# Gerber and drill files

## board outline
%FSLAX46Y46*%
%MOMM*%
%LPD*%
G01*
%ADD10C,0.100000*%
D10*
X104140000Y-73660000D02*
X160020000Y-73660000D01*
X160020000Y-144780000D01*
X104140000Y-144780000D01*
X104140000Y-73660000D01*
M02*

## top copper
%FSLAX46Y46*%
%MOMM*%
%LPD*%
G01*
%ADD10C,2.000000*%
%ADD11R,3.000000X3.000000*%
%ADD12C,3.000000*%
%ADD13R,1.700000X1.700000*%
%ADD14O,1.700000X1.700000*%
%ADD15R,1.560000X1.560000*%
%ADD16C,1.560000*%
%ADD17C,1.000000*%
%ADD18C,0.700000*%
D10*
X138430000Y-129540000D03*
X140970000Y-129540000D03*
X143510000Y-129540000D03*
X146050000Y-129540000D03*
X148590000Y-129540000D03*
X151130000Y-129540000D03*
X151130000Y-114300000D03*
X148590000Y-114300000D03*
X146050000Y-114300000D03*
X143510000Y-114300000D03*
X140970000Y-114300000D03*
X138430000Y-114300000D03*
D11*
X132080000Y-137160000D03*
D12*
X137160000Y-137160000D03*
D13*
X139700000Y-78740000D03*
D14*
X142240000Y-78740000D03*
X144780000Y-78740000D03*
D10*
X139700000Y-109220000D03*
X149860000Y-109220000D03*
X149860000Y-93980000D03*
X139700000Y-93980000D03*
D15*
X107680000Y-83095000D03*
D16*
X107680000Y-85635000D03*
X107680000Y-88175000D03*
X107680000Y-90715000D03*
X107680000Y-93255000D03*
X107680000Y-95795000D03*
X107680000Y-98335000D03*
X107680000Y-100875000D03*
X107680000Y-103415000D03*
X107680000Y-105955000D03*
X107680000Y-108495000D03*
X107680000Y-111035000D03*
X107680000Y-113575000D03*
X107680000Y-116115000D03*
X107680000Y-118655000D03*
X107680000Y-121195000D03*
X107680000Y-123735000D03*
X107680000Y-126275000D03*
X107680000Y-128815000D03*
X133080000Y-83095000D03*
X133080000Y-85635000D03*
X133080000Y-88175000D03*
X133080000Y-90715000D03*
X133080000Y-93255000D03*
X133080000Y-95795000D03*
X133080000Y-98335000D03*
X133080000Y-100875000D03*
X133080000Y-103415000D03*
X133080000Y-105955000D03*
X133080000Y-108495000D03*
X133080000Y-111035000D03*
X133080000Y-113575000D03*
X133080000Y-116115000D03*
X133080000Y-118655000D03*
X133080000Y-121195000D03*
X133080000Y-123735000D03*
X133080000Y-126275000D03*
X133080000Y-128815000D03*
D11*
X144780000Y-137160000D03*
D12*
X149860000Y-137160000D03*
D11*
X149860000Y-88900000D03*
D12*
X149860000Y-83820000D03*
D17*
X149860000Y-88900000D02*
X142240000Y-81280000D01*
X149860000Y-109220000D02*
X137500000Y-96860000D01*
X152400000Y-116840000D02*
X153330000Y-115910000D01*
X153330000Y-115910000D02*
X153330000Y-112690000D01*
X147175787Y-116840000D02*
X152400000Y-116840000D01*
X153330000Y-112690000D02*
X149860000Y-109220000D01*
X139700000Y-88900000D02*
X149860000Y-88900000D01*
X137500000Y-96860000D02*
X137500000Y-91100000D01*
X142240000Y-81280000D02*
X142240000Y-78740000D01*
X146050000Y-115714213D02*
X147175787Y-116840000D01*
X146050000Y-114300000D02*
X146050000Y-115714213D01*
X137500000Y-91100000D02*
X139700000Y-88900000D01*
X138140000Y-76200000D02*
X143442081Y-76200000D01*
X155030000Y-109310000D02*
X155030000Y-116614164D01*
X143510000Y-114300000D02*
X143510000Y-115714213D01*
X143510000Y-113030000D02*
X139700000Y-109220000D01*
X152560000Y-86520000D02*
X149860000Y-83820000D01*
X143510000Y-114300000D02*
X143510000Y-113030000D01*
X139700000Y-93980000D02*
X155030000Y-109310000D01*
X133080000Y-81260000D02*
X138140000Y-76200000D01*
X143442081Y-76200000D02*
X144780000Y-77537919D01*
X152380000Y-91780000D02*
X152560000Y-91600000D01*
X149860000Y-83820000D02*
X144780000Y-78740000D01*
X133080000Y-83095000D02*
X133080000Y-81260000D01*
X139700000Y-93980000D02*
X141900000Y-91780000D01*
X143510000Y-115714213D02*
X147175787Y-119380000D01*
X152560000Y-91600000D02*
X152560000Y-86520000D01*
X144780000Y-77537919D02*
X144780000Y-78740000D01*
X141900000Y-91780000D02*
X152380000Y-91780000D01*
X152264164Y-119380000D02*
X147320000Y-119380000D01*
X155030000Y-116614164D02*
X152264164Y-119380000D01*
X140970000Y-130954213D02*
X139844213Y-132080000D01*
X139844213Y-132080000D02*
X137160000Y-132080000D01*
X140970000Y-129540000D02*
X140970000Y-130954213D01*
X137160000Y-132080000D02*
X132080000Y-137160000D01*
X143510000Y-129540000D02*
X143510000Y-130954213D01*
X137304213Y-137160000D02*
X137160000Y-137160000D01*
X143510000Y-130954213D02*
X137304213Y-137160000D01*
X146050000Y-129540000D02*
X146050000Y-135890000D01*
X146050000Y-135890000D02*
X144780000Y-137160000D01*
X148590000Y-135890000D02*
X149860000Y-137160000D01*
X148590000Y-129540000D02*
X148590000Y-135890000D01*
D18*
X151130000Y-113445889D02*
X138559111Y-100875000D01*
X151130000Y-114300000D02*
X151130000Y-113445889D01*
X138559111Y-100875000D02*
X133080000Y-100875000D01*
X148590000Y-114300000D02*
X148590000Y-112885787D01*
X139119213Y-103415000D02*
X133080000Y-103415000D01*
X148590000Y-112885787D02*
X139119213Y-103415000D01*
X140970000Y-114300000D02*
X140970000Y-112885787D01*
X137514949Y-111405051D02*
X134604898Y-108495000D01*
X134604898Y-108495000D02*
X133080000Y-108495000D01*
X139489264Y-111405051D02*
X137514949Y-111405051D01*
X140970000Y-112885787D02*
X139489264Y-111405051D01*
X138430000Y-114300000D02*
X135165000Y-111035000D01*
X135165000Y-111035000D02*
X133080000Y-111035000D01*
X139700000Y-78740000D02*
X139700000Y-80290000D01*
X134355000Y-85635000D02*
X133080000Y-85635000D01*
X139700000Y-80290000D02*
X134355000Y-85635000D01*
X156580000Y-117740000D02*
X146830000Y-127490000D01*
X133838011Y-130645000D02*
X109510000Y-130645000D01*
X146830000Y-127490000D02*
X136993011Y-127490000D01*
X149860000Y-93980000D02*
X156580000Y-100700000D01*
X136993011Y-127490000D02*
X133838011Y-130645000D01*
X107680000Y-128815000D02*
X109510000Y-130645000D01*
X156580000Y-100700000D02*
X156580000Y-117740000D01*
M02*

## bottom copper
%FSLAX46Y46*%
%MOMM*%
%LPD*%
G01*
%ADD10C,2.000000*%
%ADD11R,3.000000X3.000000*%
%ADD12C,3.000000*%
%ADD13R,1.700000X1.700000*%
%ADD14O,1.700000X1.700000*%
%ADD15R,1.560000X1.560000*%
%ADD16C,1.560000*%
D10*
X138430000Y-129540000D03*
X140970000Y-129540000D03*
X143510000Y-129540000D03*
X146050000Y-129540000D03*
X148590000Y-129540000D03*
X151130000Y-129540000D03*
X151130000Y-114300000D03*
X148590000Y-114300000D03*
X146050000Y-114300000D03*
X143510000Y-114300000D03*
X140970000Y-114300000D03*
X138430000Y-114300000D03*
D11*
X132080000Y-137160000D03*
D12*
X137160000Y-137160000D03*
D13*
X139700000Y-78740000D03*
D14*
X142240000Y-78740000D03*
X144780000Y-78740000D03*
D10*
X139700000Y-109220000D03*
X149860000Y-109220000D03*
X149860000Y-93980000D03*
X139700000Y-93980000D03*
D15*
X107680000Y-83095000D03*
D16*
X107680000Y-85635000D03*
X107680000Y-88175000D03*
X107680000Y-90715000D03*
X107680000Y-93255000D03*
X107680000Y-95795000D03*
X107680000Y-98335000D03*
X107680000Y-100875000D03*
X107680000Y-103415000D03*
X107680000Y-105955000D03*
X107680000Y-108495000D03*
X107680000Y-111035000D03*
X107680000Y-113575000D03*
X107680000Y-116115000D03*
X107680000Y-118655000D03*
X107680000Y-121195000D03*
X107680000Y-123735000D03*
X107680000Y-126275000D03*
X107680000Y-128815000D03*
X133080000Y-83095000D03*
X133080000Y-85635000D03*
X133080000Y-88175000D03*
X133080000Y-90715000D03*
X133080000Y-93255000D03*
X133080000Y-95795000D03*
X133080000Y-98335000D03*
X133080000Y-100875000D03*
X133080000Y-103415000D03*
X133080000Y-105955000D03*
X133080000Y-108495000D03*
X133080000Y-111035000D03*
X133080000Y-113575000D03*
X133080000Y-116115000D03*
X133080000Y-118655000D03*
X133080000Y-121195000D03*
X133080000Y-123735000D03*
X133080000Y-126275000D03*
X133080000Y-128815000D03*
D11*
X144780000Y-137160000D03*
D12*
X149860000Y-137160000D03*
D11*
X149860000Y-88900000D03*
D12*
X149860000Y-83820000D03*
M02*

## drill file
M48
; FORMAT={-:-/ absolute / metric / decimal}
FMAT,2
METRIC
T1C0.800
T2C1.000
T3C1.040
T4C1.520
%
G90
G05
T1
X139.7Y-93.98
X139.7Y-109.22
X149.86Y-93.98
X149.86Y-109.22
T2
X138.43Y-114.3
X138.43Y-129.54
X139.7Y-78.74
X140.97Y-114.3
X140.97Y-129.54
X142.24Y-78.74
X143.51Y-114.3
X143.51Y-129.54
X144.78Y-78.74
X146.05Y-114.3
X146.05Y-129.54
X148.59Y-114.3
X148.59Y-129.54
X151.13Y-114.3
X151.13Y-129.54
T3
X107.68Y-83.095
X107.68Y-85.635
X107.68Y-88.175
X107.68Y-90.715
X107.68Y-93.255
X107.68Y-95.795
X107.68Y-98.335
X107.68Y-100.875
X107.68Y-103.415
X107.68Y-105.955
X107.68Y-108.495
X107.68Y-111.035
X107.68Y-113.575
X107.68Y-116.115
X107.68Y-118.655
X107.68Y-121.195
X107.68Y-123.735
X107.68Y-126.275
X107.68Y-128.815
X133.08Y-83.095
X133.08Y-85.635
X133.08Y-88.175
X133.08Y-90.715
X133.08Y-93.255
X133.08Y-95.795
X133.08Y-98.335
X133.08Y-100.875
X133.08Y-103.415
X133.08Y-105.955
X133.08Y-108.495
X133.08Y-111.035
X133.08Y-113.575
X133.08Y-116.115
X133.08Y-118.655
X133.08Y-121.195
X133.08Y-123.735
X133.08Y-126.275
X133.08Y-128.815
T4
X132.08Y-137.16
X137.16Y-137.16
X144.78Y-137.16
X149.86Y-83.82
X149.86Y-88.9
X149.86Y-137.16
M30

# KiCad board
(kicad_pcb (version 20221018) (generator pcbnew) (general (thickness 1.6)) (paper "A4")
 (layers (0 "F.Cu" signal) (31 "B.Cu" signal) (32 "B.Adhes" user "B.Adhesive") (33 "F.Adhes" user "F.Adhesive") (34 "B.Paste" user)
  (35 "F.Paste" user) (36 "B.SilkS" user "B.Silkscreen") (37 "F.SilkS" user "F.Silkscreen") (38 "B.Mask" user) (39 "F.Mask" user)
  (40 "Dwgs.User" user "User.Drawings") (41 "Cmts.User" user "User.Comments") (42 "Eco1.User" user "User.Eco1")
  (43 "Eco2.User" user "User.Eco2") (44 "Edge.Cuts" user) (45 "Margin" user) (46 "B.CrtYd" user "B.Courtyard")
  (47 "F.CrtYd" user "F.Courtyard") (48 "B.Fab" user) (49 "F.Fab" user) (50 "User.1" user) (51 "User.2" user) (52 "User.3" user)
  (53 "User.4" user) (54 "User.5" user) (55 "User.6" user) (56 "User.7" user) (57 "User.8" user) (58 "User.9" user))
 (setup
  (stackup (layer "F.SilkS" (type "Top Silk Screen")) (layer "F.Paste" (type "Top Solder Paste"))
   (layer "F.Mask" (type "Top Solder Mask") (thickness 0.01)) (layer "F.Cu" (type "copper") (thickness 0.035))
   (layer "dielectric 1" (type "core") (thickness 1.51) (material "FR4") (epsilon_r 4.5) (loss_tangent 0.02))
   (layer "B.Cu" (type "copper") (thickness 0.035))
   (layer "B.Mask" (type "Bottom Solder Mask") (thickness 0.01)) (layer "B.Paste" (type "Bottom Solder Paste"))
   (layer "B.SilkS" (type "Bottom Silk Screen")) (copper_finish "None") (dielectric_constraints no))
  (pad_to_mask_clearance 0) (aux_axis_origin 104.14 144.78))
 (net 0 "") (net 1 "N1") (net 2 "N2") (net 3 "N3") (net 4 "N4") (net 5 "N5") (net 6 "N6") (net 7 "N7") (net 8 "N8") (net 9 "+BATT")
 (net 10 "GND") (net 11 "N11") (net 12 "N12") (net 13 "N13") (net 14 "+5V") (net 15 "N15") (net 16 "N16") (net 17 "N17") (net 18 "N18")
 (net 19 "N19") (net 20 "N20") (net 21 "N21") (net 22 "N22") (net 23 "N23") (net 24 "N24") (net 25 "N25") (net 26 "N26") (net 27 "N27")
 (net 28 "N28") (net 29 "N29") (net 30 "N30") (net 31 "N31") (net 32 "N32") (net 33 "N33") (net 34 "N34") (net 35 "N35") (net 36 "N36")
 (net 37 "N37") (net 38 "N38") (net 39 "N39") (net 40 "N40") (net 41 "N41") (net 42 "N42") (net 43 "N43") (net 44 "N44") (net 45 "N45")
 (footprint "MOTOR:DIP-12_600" (layer "F.Cu") (at 144.78 121.92)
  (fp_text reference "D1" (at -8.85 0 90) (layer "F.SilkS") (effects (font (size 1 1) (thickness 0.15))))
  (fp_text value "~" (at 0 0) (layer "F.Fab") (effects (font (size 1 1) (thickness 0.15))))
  (pad "1" thru_hole circle (at -6.35 7.62) (size 2 2) (drill 1) (layers "*.Cu" "*.Mask") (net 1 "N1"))
  (pad "2" thru_hole circle (at -3.81 7.62) (size 2 2) (drill 1) (layers "*.Cu" "*.Mask") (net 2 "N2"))
  (pad "3" thru_hole circle (at -1.27 7.62) (size 2 2) (drill 1) (layers "*.Cu" "*.Mask") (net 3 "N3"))
  (pad "4" thru_hole circle (at 1.27 7.62) (size 2 2) (drill 1) (layers "*.Cu" "*.Mask") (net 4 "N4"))
  (pad "5" thru_hole circle (at 3.81 7.62) (size 2 2) (drill 1) (layers "*.Cu" "*.Mask") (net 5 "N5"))
  (pad "6" thru_hole circle (at 6.35 7.62) (size 2 2) (drill 1) (layers "*.Cu" "*.Mask") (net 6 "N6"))
  (pad "7" thru_hole circle (at 6.35 -7.62) (size 2 2) (drill 1) (layers "*.Cu" "*.Mask") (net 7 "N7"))
  (pad "8" thru_hole circle (at 3.81 -7.62) (size 2 2) (drill 1) (layers "*.Cu" "*.Mask") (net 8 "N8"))
  (pad "9" thru_hole circle (at 1.27 -7.62) (size 2 2) (drill 1) (layers "*.Cu" "*.Mask") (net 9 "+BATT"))
  (pad "10" thru_hole circle (at -1.27 -7.62) (size 2 2) (drill 1) (layers "*.Cu" "*.Mask") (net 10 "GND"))
  (pad "11" thru_hole circle (at -3.81 -7.62) (size 2 2) (drill 1) (layers "*.Cu" "*.Mask") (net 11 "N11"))
  (pad "12" thru_hole circle (at -6.35 -7.62) (size 2 2) (drill 1) (layers "*.Cu" "*.Mask") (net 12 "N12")))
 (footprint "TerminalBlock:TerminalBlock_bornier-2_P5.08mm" (layer "F.Cu") (at 132.08 137.16)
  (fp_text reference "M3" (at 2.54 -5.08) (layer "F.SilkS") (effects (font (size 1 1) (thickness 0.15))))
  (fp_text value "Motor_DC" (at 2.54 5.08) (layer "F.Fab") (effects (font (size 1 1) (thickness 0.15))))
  (pad "1" thru_hole rect (at 0 0) (size 3 3) (drill 1.52) (layers "*.Cu" "*.Mask") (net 2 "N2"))
  (pad "2" thru_hole circle (at 5.08 0) (size 3 3) (drill 1.52) (layers "*.Cu" "*.Mask") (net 3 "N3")))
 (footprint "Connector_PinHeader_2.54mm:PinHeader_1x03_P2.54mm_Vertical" (layer "F.Cu") (at 139.7 78.74 90)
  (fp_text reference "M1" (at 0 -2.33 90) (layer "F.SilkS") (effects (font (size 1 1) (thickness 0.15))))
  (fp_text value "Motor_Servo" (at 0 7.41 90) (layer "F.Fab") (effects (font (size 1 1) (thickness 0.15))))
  (pad "1" thru_hole rect (at 0 0 90) (size 1.7 1.7) (drill 1) (layers "*.Cu" "*.Mask") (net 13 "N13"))
  (pad "2" thru_hole oval (at 0 2.54 90) (size 1.7 1.7) (drill 1) (layers "*.Cu" "*.Mask") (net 9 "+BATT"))
  (pad "3" thru_hole oval (at 0 5.08 90) (size 1.7 1.7) (drill 1) (layers "*.Cu" "*.Mask") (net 10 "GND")))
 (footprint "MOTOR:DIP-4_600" (layer "F.Cu") (at 144.78 101.6)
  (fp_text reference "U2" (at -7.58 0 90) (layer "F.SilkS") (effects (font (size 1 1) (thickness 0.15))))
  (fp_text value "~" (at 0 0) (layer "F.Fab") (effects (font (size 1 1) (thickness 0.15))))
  (pad "1" thru_hole circle (at -5.08 7.62) (size 2 2) (drill 0.8) (layers "*.Cu" "*.Mask") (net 10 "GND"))
  (pad "2" thru_hole circle (at 5.08 7.62) (size 2 2) (drill 0.8) (layers "*.Cu" "*.Mask") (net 9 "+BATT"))
  (pad "3" thru_hole circle (at 5.08 -7.62) (size 2 2) (drill 0.8) (layers "*.Cu" "*.Mask") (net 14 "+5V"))
  (pad "4" thru_hole circle (at -5.08 -7.62) (size 2 2) (drill 0.8) (layers "*.Cu" "*.Mask") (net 10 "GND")))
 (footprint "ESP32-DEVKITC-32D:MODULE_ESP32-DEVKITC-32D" (layer "F.Cu") (at 120.38 102.855)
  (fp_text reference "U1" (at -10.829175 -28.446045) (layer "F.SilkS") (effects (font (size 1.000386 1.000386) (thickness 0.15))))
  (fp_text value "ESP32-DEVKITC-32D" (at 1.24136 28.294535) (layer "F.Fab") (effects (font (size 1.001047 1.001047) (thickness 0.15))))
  (pad "J2-1" thru_hole rect (at -12.7 -19.76) (size 1.56 1.56) (drill 1.04) (layers "*.Cu" "*.Mask") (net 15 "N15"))
  (pad "J2-2" thru_hole circle (at -12.7 -17.22) (size 1.56 1.56) (drill 1.04) (layers "*.Cu" "*.Mask") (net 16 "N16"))
  (pad "J2-3" thru_hole circle (at -12.7 -14.68) (size 1.56 1.56) (drill 1.04) (layers "*.Cu" "*.Mask") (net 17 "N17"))
  (pad "J2-4" thru_hole circle (at -12.7 -12.14) (size 1.56 1.56) (drill 1.04) (layers "*.Cu" "*.Mask") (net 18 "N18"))
  (pad "J2-5" thru_hole circle (at -12.7 -9.6) (size 1.56 1.56) (drill 1.04) (layers "*.Cu" "*.Mask") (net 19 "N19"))
  (pad "J2-6" thru_hole circle (at -12.7 -7.06) (size 1.56 1.56) (drill 1.04) (layers "*.Cu" "*.Mask") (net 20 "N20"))
  (pad "J2-7" thru_hole circle (at -12.7 -4.52) (size 1.56 1.56) (drill 1.04) (layers "*.Cu" "*.Mask") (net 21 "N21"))
  (pad "J2-8" thru_hole circle (at -12.7 -1.98) (size 1.56 1.56) (drill 1.04) (layers "*.Cu" "*.Mask") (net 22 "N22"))
  (pad "J2-9" thru_hole circle (at -12.7 0.56) (size 1.56 1.56) (drill 1.04) (layers "*.Cu" "*.Mask") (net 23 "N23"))
  (pad "J2-10" thru_hole circle (at -12.7 3.1) (size 1.56 1.56) (drill 1.04) (layers "*.Cu" "*.Mask") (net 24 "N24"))
  (pad "J2-11" thru_hole circle (at -12.7 5.64) (size 1.56 1.56) (drill 1.04) (layers "*.Cu" "*.Mask") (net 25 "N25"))
  (pad "J2-12" thru_hole circle (at -12.7 8.18) (size 1.56 1.56) (drill 1.04) (layers "*.Cu" "*.Mask") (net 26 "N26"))
  (pad "J2-13" thru_hole circle (at -12.7 10.72) (size 1.56 1.56) (drill 1.04) (layers "*.Cu" "*.Mask") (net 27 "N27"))
  (pad "J2-14" thru_hole circle (at -12.7 13.26) (size 1.56 1.56) (drill 1.04) (layers "*.Cu" "*.Mask") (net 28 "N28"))
  (pad "J2-15" thru_hole circle (at -12.7 15.8) (size 1.56 1.56) (drill 1.04) (layers "*.Cu" "*.Mask") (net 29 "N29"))
  (pad "J2-16" thru_hole circle (at -12.7 18.34) (size 1.56 1.56) (drill 1.04) (layers "*.Cu" "*.Mask") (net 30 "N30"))
  (pad "J2-17" thru_hole circle (at -12.7 20.88) (size 1.56 1.56) (drill 1.04) (layers "*.Cu" "*.Mask") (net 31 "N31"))
  (pad "J2-18" thru_hole circle (at -12.7 23.42) (size 1.56 1.56) (drill 1.04) (layers "*.Cu" "*.Mask") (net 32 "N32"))
  (pad "J2-19" thru_hole circle (at -12.7 25.96) (size 1.56 1.56) (drill 1.04) (layers "*.Cu" "*.Mask") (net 14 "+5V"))
  (pad "J3-1" thru_hole circle (at 12.7 -19.76) (size 1.56 1.56) (drill 1.04) (layers "*.Cu" "*.Mask") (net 10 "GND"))
  (pad "J3-2" thru_hole circle (at 12.7 -17.22) (size 1.56 1.56) (drill 1.04) (layers "*.Cu" "*.Mask") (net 13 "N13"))
  (pad "J3-3" thru_hole circle (at 12.7 -14.68) (size 1.56 1.56) (drill 1.04) (layers "*.Cu" "*.Mask") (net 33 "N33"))
  (pad "J3-4" thru_hole circle (at 12.7 -12.14) (size 1.56 1.56) (drill 1.04) (layers "*.Cu" "*.Mask") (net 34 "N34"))
  (pad "J3-5" thru_hole circle (at 12.7 -9.6) (size 1.56 1.56) (drill 1.04) (layers "*.Cu" "*.Mask") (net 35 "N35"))
  (pad "J3-6" thru_hole circle (at 12.7 -7.06) (size 1.56 1.56) (drill 1.04) (layers "*.Cu" "*.Mask") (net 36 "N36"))
  (pad "J3-7" thru_hole circle (at 12.7 -4.52) (size 1.56 1.56) (drill 1.04) (layers "*.Cu" "*.Mask") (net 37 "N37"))
  (pad "J3-8" thru_hole circle (at 12.7 -1.98) (size 1.56 1.56) (drill 1.04) (layers "*.Cu" "*.Mask") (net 7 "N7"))
  (pad "J3-9" thru_hole circle (at 12.7 0.56) (size 1.56 1.56) (drill 1.04) (layers "*.Cu" "*.Mask") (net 8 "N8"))
  (pad "J3-10" thru_hole circle (at 12.7 3.1) (size 1.56 1.56) (drill 1.04) (layers "*.Cu" "*.Mask") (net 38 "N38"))
  (pad "J3-11" thru_hole circle (at 12.7 5.64) (size 1.56 1.56) (drill 1.04) (layers "*.Cu" "*.Mask") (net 11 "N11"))
  (pad "J3-12" thru_hole circle (at 12.7 8.18) (size 1.56 1.56) (drill 1.04) (layers "*.Cu" "*.Mask") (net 12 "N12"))
  (pad "J3-13" thru_hole circle (at 12.7 10.72) (size 1.56 1.56) (drill 1.04) (layers "*.Cu" "*.Mask") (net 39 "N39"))
  (pad "J3-14" thru_hole circle (at 12.7 13.26) (size 1.56 1.56) (drill 1.04) (layers "*.Cu" "*.Mask") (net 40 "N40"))
  (pad "J3-15" thru_hole circle (at 12.7 15.8) (size 1.56 1.56) (drill 1.04) (layers "*.Cu" "*.Mask") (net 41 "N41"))
  (pad "J3-16" thru_hole circle (at 12.7 18.34) (size 1.56 1.56) (drill 1.04) (layers "*.Cu" "*.Mask") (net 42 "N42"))
  (pad "J3-17" thru_hole circle (at 12.7 20.88) (size 1.56 1.56) (drill 1.04) (layers "*.Cu" "*.Mask") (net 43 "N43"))
  (pad "J3-18" thru_hole circle (at 12.7 23.42) (size 1.56 1.56) (drill 1.04) (layers "*.Cu" "*.Mask") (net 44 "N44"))
  (pad "J3-19" thru_hole circle (at 12.7 25.96) (size 1.56 1.56) (drill 1.04) (layers "*.Cu" "*.Mask") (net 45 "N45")))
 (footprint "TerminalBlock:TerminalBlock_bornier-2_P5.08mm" (layer "F.Cu") (at 144.78 137.16)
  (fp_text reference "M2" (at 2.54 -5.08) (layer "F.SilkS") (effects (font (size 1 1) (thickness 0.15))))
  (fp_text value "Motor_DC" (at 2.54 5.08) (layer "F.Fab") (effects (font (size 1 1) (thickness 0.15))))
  (pad "1" thru_hole rect (at 0 0) (size 3 3) (drill 1.52) (layers "*.Cu" "*.Mask") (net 4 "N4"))
  (pad "2" thru_hole circle (at 5.08 0) (size 3 3) (drill 1.52) (layers "*.Cu" "*.Mask") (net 5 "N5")))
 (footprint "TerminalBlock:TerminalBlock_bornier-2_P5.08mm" (layer "F.Cu") (at 149.86 88.9 90)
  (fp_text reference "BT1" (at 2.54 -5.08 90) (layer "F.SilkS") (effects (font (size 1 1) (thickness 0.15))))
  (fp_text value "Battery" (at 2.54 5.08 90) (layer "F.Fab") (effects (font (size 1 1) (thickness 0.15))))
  (pad "1" thru_hole rect (at 0 0 90) (size 3 3) (drill 1.52) (layers "*.Cu" "*.Mask") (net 9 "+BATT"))
  (pad "2" thru_hole circle (at 5.08 0 90) (size 3 3) (drill 1.52) (layers "*.Cu" "*.Mask") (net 10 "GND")))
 (gr_rect (start 104.14 73.66) (end 160.02 144.78) (stroke (width 0.1) (type default)) (fill none) (layer "Edge.Cuts"))
 (segment (start 149.86 88.9) (end 142.24 81.28) (width 1) (layer "F.Cu") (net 9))
 (segment (start 149.86 109.22) (end 137.5 96.86) (width 1) (layer "F.Cu") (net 9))
 (segment (start 152.4 116.84) (end 153.33 115.91) (width 1) (layer "F.Cu") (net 9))
 (segment (start 153.33 115.91) (end 153.33 112.69) (width 1) (layer "F.Cu") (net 9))
 (segment (start 147.175787 116.84) (end 152.4 116.84) (width 1) (layer "F.Cu") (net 9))
 (segment (start 153.33 112.69) (end 149.86 109.22) (width 1) (layer "F.Cu") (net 9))
 (segment (start 139.7 88.9) (end 149.86 88.9) (width 1) (layer "F.Cu") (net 9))
 (segment (start 137.5 96.86) (end 137.5 91.1) (width 1) (layer "F.Cu") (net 9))
 (segment (start 142.24 81.28) (end 142.24 78.74) (width 1) (layer "F.Cu") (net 9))
 (segment (start 146.05 115.714213) (end 147.175787 116.84) (width 1) (layer "F.Cu") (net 9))
 (segment (start 146.05 114.3) (end 146.05 115.714213) (width 1) (layer "F.Cu") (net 9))
 (segment (start 137.5 91.1) (end 139.7 88.9) (width 1) (layer "F.Cu") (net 9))
 (segment (start 138.14 76.2) (end 143.442081 76.2) (width 1) (layer "F.Cu") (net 10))
 (segment (start 155.03 109.31) (end 155.03 116.614164) (width 1) (layer "F.Cu") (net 10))
 (segment (start 143.51 114.3) (end 143.51 115.714213) (width 1) (layer "F.Cu") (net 10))
 (segment (start 143.51 113.03) (end 139.7 109.22) (width 1) (layer "F.Cu") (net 10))
 (segment (start 152.56 86.52) (end 149.86 83.82) (width 1) (layer "F.Cu") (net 10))
 (segment (start 143.51 114.3) (end 143.51 113.03) (width 1) (layer "F.Cu") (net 10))
 (segment (start 139.7 93.98) (end 155.03 109.31) (width 1) (layer "F.Cu") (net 10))
 (segment (start 133.08 81.26) (end 138.14 76.2) (width 1) (layer "F.Cu") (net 10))
 (segment (start 143.442081 76.2) (end 144.78 77.537919) (width 1) (layer "F.Cu") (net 10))
 (segment (start 152.38 91.78) (end 152.56 91.6) (width 1) (layer "F.Cu") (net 10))
 (segment (start 149.86 83.82) (end 144.78 78.74) (width 1) (layer "F.Cu") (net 10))
 (segment (start 133.08 83.095) (end 133.08 81.26) (width 1) (layer "F.Cu") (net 10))
 (segment (start 139.7 93.98) (end 141.9 91.78) (width 1) (layer "F.Cu") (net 10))
 (segment (start 143.51 115.714213) (end 147.175787 119.38) (width 1) (layer "F.Cu") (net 10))
 (segment (start 152.56 91.6) (end 152.56 86.52) (width 1) (layer "F.Cu") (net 10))
 (segment (start 144.78 77.537919) (end 144.78 78.74) (width 1) (layer "F.Cu") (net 10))
 (segment (start 141.9 91.78) (end 152.38 91.78) (width 1) (layer "F.Cu") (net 10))
 (segment (start 152.264164 119.38) (end 147.32 119.38) (width 1) (layer "F.Cu") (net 10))
 (segment (start 155.03 116.614164) (end 152.264164 119.38) (width 1) (layer "F.Cu") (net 10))
 (segment (start 140.97 130.954213) (end 139.844213 132.08) (width 1) (layer "F.Cu") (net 2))
 (segment (start 139.844213 132.08) (end 137.16 132.08) (width 1) (layer "F.Cu") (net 2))
 (segment (start 140.97 129.54) (end 140.97 130.954213) (width 1) (layer "F.Cu") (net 2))
 (segment (start 137.16 132.08) (end 132.08 137.16) (width 1) (layer "F.Cu") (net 2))
 (segment (start 143.51 129.54) (end 143.51 130.954213) (width 1) (layer "F.Cu") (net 3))
 (segment (start 137.304213 137.16) (end 137.16 137.16) (width 1) (layer "F.Cu") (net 3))
 (segment (start 143.51 130.954213) (end 137.304213 137.16) (width 1) (layer "F.Cu") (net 3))
 (segment (start 146.05 129.54) (end 146.05 135.89) (width 1) (layer "F.Cu") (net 4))
 (segment (start 146.05 135.89) (end 144.78 137.16) (width 1) (layer "F.Cu") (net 4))
 (segment (start 148.59 135.89) (end 149.86 137.16) (width 1) (layer "F.Cu") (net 5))
 (segment (start 148.59 129.54) (end 148.59 135.89) (width 1) (layer "F.Cu") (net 5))
 (segment (start 151.13 113.445889) (end 138.559111 100.875) (width 0.7) (layer "F.Cu") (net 7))
 (segment (start 151.13 114.3) (end 151.13 113.445889) (width 0.7) (layer "F.Cu") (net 7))
 (segment (start 138.559111 100.875) (end 133.08 100.875) (width 0.7) (layer "F.Cu") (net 7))
 (segment (start 148.59 114.3) (end 148.59 112.885787) (width 0.7) (layer "F.Cu") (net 8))
 (segment (start 139.119213 103.415) (end 133.08 103.415) (width 0.7) (layer "F.Cu") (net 8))
 (segment (start 148.59 112.885787) (end 139.119213 103.415) (width 0.7) (layer "F.Cu") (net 8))
 (segment (start 140.97 114.3) (end 140.97 112.885787) (width 0.7) (layer "F.Cu") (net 11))
 (segment (start 137.514949 111.405051) (end 134.604898 108.495) (width 0.7) (layer "F.Cu") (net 11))
 (segment (start 134.604898 108.495) (end 133.08 108.495) (width 0.7) (layer "F.Cu") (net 11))
 (segment (start 139.489264 111.405051) (end 137.514949 111.405051) (width 0.7) (layer "F.Cu") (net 11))
 (segment (start 140.97 112.885787) (end 139.489264 111.405051) (width 0.7) (layer "F.Cu") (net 11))
 (segment (start 138.43 114.3) (end 135.165 111.035) (width 0.7) (layer "F.Cu") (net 12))
 (segment (start 135.165 111.035) (end 133.08 111.035) (width 0.7) (layer "F.Cu") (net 12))
 (segment (start 139.7 78.74) (end 139.7 80.29) (width 0.7) (layer "F.Cu") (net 13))
 (segment (start 134.355 85.635) (end 133.08 85.635) (width 0.7) (layer "F.Cu") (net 13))
 (segment (start 139.7 80.29) (end 134.355 85.635) (width 0.7) (layer "F.Cu") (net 13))
 (segment (start 156.58 117.74) (end 146.83 127.49) (width 0.7) (layer "F.Cu") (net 14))
 (segment (start 133.838011 130.645) (end 109.51 130.645) (width 0.7) (layer "F.Cu") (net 14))
 (segment (start 146.83 127.49) (end 136.993011 127.49) (width 0.7) (layer "F.Cu") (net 14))
 (segment (start 149.86 93.98) (end 156.58 100.7) (width 0.7) (layer "F.Cu") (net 14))
 (segment (start 136.993011 127.49) (end 133.838011 130.645) (width 0.7) (layer "F.Cu") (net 14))
 (segment (start 107.68 128.815) (end 109.51 130.645) (width 0.7) (layer "F.Cu") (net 14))
 (segment (start 156.58 100.7) (end 156.58 117.74) (width 0.7) (layer "F.Cu") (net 14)))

